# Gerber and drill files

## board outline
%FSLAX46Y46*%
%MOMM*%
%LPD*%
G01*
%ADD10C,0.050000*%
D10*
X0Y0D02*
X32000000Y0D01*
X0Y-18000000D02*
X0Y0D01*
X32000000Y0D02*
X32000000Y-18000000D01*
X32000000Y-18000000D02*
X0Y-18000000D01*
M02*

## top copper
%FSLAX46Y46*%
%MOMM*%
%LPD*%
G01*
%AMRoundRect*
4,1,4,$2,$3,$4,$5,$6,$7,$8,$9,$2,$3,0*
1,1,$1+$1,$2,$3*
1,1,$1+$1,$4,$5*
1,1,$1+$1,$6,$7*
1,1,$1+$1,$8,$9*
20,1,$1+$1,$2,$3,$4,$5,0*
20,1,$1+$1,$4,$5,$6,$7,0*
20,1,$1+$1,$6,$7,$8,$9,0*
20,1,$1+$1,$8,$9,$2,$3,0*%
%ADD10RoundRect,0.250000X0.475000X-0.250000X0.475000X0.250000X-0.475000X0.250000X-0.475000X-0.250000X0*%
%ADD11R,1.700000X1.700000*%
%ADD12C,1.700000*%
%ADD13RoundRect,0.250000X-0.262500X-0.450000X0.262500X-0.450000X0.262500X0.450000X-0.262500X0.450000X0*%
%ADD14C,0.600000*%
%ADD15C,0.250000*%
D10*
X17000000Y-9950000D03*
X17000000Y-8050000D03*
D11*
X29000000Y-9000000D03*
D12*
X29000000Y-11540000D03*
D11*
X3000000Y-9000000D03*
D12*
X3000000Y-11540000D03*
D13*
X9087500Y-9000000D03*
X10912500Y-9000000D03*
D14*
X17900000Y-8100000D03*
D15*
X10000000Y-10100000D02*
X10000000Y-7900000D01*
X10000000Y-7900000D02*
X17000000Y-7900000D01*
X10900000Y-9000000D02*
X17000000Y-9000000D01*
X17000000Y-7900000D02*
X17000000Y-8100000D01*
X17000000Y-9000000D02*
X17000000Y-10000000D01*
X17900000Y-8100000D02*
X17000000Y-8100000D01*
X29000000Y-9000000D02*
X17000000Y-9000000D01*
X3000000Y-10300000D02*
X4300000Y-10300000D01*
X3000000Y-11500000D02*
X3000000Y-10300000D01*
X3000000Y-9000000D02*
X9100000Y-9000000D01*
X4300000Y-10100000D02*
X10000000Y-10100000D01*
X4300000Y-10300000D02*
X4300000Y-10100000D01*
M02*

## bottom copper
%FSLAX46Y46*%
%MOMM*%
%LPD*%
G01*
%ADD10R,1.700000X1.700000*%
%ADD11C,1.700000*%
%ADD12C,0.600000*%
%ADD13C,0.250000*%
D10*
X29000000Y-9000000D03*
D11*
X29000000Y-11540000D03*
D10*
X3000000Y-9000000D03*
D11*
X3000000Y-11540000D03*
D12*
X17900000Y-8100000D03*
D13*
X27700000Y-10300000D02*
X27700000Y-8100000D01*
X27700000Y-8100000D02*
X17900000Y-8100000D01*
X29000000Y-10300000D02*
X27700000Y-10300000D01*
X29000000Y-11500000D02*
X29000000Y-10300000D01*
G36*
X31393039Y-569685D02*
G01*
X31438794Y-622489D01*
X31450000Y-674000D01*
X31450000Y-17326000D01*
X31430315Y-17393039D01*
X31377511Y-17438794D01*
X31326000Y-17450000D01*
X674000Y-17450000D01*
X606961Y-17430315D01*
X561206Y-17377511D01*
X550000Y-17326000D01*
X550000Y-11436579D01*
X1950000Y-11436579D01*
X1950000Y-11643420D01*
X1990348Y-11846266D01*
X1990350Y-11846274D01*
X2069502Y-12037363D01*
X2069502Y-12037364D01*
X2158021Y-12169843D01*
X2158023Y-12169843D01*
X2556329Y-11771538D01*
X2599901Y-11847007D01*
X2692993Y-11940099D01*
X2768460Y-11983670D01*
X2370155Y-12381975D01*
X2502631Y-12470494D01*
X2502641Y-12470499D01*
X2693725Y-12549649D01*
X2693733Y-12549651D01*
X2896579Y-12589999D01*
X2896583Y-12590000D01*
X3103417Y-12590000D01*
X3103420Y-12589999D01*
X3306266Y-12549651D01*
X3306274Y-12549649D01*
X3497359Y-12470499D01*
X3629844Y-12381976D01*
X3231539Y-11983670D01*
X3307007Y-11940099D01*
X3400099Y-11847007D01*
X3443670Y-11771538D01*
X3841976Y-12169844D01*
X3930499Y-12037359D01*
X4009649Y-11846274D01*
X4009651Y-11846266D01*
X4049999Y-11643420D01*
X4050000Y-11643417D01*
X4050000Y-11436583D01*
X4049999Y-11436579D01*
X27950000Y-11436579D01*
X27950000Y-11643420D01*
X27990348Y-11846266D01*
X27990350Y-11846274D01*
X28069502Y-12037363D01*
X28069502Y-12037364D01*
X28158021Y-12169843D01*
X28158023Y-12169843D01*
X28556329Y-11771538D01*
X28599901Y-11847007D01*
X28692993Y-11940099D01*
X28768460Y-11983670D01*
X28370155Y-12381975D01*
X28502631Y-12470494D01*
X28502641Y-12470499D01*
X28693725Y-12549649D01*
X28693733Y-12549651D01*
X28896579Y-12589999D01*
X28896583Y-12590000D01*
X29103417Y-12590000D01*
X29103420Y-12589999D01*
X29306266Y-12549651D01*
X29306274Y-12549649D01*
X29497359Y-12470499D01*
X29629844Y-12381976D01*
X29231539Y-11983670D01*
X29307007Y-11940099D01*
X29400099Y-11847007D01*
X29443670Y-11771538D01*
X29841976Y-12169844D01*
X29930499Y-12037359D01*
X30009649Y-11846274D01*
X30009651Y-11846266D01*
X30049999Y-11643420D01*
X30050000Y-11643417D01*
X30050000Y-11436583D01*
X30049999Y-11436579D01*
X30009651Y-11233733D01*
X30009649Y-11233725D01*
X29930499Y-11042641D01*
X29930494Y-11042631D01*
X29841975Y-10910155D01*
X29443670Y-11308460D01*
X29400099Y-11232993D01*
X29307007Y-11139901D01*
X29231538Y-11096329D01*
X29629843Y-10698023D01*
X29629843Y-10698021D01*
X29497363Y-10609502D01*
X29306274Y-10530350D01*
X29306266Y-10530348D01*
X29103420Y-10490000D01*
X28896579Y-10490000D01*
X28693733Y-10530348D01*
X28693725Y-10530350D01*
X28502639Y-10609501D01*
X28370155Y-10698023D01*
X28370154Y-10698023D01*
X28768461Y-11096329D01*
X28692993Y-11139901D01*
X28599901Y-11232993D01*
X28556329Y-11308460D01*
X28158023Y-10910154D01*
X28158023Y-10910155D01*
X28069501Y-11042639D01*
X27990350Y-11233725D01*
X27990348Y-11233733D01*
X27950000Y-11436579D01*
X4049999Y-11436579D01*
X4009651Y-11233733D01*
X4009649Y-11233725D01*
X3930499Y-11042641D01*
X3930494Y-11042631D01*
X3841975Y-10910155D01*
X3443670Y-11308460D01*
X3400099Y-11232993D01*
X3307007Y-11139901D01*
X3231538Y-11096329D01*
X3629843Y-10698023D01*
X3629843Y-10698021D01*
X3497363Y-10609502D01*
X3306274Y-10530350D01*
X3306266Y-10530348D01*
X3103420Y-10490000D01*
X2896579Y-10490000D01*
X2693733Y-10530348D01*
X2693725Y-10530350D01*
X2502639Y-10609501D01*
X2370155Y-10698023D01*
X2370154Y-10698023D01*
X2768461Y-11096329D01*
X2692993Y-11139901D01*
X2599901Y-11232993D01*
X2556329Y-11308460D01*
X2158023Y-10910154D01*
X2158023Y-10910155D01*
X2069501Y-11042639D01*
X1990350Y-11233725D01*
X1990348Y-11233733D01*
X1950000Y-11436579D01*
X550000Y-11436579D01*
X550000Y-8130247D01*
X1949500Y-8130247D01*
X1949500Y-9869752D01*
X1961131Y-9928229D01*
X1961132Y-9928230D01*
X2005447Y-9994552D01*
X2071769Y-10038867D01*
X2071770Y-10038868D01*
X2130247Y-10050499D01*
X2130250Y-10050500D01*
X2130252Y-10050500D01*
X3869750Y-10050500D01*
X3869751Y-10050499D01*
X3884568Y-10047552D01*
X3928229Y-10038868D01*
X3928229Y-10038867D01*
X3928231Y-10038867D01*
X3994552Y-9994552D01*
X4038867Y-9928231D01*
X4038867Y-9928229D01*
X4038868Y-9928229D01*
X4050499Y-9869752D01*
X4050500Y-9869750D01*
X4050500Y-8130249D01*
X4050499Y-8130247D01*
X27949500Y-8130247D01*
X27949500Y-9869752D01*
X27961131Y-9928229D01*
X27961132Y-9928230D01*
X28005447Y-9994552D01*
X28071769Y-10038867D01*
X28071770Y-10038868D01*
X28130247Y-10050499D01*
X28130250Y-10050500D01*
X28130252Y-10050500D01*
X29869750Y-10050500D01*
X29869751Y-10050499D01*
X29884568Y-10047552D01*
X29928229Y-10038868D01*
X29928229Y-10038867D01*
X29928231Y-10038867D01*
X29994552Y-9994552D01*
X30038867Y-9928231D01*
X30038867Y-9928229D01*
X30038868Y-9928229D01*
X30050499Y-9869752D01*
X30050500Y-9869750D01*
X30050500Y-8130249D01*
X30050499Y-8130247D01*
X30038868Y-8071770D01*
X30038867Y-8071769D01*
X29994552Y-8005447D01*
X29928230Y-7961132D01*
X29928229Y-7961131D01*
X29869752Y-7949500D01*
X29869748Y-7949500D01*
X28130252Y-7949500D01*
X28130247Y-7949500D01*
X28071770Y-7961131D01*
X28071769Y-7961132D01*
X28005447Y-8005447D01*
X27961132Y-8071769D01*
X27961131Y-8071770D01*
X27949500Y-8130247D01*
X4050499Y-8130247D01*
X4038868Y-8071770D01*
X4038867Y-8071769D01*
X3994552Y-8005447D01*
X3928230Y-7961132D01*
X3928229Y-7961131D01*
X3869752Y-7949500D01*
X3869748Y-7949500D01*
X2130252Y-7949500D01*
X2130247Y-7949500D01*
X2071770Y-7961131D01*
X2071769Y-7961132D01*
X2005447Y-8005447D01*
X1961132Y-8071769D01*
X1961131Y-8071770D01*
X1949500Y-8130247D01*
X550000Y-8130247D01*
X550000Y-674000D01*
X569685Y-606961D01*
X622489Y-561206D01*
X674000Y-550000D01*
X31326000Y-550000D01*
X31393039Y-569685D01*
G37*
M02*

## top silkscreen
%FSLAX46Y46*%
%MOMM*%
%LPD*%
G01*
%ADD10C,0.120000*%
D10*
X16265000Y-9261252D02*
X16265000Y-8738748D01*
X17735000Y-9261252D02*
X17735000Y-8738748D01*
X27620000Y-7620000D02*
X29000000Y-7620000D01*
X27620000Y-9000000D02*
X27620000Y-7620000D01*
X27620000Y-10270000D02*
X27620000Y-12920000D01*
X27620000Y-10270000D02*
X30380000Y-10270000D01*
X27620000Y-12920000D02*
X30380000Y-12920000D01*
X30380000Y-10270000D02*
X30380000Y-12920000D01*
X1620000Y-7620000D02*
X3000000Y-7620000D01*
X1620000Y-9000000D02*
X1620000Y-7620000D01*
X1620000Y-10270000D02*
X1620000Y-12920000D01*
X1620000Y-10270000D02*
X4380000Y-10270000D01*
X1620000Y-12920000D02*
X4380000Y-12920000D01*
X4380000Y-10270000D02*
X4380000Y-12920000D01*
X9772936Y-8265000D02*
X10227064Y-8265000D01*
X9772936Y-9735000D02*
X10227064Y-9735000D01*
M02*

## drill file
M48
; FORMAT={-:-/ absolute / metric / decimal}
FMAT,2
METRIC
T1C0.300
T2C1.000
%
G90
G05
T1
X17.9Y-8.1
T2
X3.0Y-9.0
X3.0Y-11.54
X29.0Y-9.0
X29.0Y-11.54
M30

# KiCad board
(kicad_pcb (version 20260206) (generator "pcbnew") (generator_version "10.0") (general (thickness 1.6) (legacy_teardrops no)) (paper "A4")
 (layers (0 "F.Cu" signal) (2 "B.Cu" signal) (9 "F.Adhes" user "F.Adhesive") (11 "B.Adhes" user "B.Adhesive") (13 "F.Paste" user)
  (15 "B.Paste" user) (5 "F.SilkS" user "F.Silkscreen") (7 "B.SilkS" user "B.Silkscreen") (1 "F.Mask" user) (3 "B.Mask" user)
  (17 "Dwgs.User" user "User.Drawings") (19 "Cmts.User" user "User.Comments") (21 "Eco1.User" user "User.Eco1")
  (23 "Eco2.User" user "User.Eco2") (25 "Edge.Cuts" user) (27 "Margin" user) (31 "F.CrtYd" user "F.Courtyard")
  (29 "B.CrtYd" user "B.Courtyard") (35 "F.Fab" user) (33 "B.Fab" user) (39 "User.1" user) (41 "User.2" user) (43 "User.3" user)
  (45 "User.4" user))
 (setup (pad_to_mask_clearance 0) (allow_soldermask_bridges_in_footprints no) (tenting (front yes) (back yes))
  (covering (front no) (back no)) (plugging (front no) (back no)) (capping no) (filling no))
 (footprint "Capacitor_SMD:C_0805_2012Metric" (layer "F.Cu") (at 17 9 90)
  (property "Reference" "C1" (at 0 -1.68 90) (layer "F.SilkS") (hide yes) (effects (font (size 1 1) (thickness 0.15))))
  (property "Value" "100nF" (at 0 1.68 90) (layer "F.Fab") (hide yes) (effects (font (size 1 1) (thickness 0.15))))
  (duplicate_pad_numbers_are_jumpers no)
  (fp_line (start -0.261252 -0.735) (end 0.261252 -0.735) (stroke (width 0.12) (type solid)) (layer "F.SilkS"))
  (fp_line (start -0.261252 0.735) (end 0.261252 0.735) (stroke (width 0.12) (type solid)) (layer "F.SilkS"))
  (pad "1" smd roundrect (at -0.95 0 90) (size 1 1.45) (layers "F.Cu" "F.Mask" "F.Paste") (roundrect_rratio 0.25) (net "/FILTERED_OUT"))
  (pad "2" smd roundrect (at 0.95 0 90) (size 1 1.45) (layers "F.Cu" "F.Mask" "F.Paste") (roundrect_rratio 0.25) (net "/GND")))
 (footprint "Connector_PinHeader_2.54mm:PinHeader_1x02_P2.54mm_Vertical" (layer "F.Cu") (at 29 9)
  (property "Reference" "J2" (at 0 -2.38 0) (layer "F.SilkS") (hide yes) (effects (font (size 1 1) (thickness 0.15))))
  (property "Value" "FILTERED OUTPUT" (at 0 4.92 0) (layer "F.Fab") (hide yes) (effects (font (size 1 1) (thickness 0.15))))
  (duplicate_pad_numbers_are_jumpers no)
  (fp_line (start -1.38 -1.38) (end 0 -1.38) (stroke (width 0.12) (type solid)) (layer "F.SilkS"))
  (fp_line (start -1.38 0) (end -1.38 -1.38) (stroke (width 0.12) (type solid)) (layer "F.SilkS"))
  (fp_line (start -1.38 1.27) (end -1.38 3.92) (stroke (width 0.12) (type solid)) (layer "F.SilkS"))
  (fp_line (start -1.38 1.27) (end 1.38 1.27) (stroke (width 0.12) (type solid)) (layer "F.SilkS"))
  (fp_line (start -1.38 3.92) (end 1.38 3.92) (stroke (width 0.12) (type solid)) (layer "F.SilkS"))
  (fp_line (start 1.38 1.27) (end 1.38 3.92) (stroke (width 0.12) (type solid)) (layer "F.SilkS"))
  (pad "1" thru_hole rect (at 0 0) (size 1.7 1.7) (drill 1) (layers "*.Cu" "*.Mask") (remove_unused_layers no) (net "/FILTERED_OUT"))
  (pad "2" thru_hole circle (at 0 2.54) (size 1.7 1.7) (drill 1) (layers "*.Cu" "*.Mask") (remove_unused_layers no) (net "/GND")))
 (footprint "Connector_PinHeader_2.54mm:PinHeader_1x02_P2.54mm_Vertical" (layer "F.Cu") (at 3 9)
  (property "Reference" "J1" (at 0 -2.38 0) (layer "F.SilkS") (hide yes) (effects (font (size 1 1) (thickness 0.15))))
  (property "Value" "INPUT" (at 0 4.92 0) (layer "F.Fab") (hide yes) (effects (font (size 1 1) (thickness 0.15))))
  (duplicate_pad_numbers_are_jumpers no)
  (fp_line (start -1.38 -1.38) (end 0 -1.38) (stroke (width 0.12) (type solid)) (layer "F.SilkS"))
  (fp_line (start -1.38 0) (end -1.38 -1.38) (stroke (width 0.12) (type solid)) (layer "F.SilkS"))
  (fp_line (start -1.38 1.27) (end -1.38 3.92) (stroke (width 0.12) (type solid)) (layer "F.SilkS"))
  (fp_line (start -1.38 1.27) (end 1.38 1.27) (stroke (width 0.12) (type solid)) (layer "F.SilkS"))
  (fp_line (start -1.38 3.92) (end 1.38 3.92) (stroke (width 0.12) (type solid)) (layer "F.SilkS"))
  (fp_line (start 1.38 1.27) (end 1.38 3.92) (stroke (width 0.12) (type solid)) (layer "F.SilkS"))
  (pad "1" thru_hole rect (at 0 0) (size 1.7 1.7) (drill 1) (layers "*.Cu" "*.Mask") (remove_unused_layers no) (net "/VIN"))
  (pad "2" thru_hole circle (at 0 2.54) (size 1.7 1.7) (drill 1) (layers "*.Cu" "*.Mask") (remove_unused_layers no) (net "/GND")))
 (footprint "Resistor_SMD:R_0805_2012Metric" (layer "F.Cu") (at 10 9)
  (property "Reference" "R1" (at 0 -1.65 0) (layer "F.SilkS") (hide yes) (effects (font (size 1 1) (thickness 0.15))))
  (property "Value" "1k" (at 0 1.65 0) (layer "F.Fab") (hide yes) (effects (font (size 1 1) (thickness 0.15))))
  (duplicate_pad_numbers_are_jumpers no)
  (fp_line (start -0.227064 -0.735) (end 0.227064 -0.735) (stroke (width 0.12) (type solid)) (layer "F.SilkS"))
  (fp_line (start -0.227064 0.735) (end 0.227064 0.735) (stroke (width 0.12) (type solid)) (layer "F.SilkS"))
  (pad "1" smd roundrect (at -0.9125 0) (size 1.025 1.4) (layers "F.Cu" "F.Mask" "F.Paste") (roundrect_rratio 0.243902) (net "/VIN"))
  (pad "2" smd roundrect (at 0.9125 0) (size 1.025 1.4) (layers "F.Cu" "F.Mask" "F.Paste") (roundrect_rratio 0.243902) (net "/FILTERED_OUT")))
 (gr_line (start 0 0) (end 32 0) (stroke (width 0.05) (type default)) (layer "Edge.Cuts"))
 (gr_line (start 0 18) (end 0 0) (stroke (width 0.05) (type default)) (layer "Edge.Cuts"))
 (gr_line (start 32 0) (end 32 18) (stroke (width 0.05) (type default)) (layer "Edge.Cuts"))
 (gr_line (start 32 18) (end 0 18) (stroke (width 0.05) (type default)) (layer "Edge.Cuts"))
 (segment (start 10 10.1) (end 10 7.9) (width 0.25) (layer "F.Cu") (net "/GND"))
 (segment (start 10 7.9) (end 17 7.9) (width 0.25) (layer "F.Cu") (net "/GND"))
 (segment (start 10.9 9) (end 17 9) (width 0.25) (layer "F.Cu") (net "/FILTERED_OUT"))
 (segment (start 17 7.9) (end 17 8.1) (width 0.25) (layer "F.Cu") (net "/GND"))
 (segment (start 17 9) (end 17 10) (width 0.25) (layer "F.Cu") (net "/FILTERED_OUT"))
 (segment (start 17.9 8.1) (end 17 8.1) (width 0.25) (layer "F.Cu") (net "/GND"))
 (segment (start 27.7 10.3) (end 27.7 8.1) (width 0.25) (layer "B.Cu") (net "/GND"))
 (segment (start 27.7 8.1) (end 17.9 8.1) (width 0.25) (layer "B.Cu") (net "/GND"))
 (segment (start 29 10.3) (end 27.7 10.3) (width 0.25) (layer "B.Cu") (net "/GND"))
 (segment (start 29 11.5) (end 29 10.3) (width 0.25) (layer "B.Cu") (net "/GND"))
 (segment (start 29 9) (end 17 9) (width 0.25) (layer "F.Cu") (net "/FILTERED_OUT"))
 (segment (start 3 10.3) (end 4.3 10.3) (width 0.25) (layer "F.Cu") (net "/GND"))
 (segment (start 3 11.5) (end 3 10.3) (width 0.25) (layer "F.Cu") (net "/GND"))
 (segment (start 3 9) (end 9.1 9) (width 0.25) (layer "F.Cu") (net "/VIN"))
 (segment (start 4.3 10.1) (end 10 10.1) (width 0.25) (layer "F.Cu") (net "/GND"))
 (segment (start 4.3 10.3) (end 4.3 10.1) (width 0.25) (layer "F.Cu") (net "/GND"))
 (via (at 17.9 8.1) (size 0.6) (drill 0.3) (layers "F.Cu" "B.Cu") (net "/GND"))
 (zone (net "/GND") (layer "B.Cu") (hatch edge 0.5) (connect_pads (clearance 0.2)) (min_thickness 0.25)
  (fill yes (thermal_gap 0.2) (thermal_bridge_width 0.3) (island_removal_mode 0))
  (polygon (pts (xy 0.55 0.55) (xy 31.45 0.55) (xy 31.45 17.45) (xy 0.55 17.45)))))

